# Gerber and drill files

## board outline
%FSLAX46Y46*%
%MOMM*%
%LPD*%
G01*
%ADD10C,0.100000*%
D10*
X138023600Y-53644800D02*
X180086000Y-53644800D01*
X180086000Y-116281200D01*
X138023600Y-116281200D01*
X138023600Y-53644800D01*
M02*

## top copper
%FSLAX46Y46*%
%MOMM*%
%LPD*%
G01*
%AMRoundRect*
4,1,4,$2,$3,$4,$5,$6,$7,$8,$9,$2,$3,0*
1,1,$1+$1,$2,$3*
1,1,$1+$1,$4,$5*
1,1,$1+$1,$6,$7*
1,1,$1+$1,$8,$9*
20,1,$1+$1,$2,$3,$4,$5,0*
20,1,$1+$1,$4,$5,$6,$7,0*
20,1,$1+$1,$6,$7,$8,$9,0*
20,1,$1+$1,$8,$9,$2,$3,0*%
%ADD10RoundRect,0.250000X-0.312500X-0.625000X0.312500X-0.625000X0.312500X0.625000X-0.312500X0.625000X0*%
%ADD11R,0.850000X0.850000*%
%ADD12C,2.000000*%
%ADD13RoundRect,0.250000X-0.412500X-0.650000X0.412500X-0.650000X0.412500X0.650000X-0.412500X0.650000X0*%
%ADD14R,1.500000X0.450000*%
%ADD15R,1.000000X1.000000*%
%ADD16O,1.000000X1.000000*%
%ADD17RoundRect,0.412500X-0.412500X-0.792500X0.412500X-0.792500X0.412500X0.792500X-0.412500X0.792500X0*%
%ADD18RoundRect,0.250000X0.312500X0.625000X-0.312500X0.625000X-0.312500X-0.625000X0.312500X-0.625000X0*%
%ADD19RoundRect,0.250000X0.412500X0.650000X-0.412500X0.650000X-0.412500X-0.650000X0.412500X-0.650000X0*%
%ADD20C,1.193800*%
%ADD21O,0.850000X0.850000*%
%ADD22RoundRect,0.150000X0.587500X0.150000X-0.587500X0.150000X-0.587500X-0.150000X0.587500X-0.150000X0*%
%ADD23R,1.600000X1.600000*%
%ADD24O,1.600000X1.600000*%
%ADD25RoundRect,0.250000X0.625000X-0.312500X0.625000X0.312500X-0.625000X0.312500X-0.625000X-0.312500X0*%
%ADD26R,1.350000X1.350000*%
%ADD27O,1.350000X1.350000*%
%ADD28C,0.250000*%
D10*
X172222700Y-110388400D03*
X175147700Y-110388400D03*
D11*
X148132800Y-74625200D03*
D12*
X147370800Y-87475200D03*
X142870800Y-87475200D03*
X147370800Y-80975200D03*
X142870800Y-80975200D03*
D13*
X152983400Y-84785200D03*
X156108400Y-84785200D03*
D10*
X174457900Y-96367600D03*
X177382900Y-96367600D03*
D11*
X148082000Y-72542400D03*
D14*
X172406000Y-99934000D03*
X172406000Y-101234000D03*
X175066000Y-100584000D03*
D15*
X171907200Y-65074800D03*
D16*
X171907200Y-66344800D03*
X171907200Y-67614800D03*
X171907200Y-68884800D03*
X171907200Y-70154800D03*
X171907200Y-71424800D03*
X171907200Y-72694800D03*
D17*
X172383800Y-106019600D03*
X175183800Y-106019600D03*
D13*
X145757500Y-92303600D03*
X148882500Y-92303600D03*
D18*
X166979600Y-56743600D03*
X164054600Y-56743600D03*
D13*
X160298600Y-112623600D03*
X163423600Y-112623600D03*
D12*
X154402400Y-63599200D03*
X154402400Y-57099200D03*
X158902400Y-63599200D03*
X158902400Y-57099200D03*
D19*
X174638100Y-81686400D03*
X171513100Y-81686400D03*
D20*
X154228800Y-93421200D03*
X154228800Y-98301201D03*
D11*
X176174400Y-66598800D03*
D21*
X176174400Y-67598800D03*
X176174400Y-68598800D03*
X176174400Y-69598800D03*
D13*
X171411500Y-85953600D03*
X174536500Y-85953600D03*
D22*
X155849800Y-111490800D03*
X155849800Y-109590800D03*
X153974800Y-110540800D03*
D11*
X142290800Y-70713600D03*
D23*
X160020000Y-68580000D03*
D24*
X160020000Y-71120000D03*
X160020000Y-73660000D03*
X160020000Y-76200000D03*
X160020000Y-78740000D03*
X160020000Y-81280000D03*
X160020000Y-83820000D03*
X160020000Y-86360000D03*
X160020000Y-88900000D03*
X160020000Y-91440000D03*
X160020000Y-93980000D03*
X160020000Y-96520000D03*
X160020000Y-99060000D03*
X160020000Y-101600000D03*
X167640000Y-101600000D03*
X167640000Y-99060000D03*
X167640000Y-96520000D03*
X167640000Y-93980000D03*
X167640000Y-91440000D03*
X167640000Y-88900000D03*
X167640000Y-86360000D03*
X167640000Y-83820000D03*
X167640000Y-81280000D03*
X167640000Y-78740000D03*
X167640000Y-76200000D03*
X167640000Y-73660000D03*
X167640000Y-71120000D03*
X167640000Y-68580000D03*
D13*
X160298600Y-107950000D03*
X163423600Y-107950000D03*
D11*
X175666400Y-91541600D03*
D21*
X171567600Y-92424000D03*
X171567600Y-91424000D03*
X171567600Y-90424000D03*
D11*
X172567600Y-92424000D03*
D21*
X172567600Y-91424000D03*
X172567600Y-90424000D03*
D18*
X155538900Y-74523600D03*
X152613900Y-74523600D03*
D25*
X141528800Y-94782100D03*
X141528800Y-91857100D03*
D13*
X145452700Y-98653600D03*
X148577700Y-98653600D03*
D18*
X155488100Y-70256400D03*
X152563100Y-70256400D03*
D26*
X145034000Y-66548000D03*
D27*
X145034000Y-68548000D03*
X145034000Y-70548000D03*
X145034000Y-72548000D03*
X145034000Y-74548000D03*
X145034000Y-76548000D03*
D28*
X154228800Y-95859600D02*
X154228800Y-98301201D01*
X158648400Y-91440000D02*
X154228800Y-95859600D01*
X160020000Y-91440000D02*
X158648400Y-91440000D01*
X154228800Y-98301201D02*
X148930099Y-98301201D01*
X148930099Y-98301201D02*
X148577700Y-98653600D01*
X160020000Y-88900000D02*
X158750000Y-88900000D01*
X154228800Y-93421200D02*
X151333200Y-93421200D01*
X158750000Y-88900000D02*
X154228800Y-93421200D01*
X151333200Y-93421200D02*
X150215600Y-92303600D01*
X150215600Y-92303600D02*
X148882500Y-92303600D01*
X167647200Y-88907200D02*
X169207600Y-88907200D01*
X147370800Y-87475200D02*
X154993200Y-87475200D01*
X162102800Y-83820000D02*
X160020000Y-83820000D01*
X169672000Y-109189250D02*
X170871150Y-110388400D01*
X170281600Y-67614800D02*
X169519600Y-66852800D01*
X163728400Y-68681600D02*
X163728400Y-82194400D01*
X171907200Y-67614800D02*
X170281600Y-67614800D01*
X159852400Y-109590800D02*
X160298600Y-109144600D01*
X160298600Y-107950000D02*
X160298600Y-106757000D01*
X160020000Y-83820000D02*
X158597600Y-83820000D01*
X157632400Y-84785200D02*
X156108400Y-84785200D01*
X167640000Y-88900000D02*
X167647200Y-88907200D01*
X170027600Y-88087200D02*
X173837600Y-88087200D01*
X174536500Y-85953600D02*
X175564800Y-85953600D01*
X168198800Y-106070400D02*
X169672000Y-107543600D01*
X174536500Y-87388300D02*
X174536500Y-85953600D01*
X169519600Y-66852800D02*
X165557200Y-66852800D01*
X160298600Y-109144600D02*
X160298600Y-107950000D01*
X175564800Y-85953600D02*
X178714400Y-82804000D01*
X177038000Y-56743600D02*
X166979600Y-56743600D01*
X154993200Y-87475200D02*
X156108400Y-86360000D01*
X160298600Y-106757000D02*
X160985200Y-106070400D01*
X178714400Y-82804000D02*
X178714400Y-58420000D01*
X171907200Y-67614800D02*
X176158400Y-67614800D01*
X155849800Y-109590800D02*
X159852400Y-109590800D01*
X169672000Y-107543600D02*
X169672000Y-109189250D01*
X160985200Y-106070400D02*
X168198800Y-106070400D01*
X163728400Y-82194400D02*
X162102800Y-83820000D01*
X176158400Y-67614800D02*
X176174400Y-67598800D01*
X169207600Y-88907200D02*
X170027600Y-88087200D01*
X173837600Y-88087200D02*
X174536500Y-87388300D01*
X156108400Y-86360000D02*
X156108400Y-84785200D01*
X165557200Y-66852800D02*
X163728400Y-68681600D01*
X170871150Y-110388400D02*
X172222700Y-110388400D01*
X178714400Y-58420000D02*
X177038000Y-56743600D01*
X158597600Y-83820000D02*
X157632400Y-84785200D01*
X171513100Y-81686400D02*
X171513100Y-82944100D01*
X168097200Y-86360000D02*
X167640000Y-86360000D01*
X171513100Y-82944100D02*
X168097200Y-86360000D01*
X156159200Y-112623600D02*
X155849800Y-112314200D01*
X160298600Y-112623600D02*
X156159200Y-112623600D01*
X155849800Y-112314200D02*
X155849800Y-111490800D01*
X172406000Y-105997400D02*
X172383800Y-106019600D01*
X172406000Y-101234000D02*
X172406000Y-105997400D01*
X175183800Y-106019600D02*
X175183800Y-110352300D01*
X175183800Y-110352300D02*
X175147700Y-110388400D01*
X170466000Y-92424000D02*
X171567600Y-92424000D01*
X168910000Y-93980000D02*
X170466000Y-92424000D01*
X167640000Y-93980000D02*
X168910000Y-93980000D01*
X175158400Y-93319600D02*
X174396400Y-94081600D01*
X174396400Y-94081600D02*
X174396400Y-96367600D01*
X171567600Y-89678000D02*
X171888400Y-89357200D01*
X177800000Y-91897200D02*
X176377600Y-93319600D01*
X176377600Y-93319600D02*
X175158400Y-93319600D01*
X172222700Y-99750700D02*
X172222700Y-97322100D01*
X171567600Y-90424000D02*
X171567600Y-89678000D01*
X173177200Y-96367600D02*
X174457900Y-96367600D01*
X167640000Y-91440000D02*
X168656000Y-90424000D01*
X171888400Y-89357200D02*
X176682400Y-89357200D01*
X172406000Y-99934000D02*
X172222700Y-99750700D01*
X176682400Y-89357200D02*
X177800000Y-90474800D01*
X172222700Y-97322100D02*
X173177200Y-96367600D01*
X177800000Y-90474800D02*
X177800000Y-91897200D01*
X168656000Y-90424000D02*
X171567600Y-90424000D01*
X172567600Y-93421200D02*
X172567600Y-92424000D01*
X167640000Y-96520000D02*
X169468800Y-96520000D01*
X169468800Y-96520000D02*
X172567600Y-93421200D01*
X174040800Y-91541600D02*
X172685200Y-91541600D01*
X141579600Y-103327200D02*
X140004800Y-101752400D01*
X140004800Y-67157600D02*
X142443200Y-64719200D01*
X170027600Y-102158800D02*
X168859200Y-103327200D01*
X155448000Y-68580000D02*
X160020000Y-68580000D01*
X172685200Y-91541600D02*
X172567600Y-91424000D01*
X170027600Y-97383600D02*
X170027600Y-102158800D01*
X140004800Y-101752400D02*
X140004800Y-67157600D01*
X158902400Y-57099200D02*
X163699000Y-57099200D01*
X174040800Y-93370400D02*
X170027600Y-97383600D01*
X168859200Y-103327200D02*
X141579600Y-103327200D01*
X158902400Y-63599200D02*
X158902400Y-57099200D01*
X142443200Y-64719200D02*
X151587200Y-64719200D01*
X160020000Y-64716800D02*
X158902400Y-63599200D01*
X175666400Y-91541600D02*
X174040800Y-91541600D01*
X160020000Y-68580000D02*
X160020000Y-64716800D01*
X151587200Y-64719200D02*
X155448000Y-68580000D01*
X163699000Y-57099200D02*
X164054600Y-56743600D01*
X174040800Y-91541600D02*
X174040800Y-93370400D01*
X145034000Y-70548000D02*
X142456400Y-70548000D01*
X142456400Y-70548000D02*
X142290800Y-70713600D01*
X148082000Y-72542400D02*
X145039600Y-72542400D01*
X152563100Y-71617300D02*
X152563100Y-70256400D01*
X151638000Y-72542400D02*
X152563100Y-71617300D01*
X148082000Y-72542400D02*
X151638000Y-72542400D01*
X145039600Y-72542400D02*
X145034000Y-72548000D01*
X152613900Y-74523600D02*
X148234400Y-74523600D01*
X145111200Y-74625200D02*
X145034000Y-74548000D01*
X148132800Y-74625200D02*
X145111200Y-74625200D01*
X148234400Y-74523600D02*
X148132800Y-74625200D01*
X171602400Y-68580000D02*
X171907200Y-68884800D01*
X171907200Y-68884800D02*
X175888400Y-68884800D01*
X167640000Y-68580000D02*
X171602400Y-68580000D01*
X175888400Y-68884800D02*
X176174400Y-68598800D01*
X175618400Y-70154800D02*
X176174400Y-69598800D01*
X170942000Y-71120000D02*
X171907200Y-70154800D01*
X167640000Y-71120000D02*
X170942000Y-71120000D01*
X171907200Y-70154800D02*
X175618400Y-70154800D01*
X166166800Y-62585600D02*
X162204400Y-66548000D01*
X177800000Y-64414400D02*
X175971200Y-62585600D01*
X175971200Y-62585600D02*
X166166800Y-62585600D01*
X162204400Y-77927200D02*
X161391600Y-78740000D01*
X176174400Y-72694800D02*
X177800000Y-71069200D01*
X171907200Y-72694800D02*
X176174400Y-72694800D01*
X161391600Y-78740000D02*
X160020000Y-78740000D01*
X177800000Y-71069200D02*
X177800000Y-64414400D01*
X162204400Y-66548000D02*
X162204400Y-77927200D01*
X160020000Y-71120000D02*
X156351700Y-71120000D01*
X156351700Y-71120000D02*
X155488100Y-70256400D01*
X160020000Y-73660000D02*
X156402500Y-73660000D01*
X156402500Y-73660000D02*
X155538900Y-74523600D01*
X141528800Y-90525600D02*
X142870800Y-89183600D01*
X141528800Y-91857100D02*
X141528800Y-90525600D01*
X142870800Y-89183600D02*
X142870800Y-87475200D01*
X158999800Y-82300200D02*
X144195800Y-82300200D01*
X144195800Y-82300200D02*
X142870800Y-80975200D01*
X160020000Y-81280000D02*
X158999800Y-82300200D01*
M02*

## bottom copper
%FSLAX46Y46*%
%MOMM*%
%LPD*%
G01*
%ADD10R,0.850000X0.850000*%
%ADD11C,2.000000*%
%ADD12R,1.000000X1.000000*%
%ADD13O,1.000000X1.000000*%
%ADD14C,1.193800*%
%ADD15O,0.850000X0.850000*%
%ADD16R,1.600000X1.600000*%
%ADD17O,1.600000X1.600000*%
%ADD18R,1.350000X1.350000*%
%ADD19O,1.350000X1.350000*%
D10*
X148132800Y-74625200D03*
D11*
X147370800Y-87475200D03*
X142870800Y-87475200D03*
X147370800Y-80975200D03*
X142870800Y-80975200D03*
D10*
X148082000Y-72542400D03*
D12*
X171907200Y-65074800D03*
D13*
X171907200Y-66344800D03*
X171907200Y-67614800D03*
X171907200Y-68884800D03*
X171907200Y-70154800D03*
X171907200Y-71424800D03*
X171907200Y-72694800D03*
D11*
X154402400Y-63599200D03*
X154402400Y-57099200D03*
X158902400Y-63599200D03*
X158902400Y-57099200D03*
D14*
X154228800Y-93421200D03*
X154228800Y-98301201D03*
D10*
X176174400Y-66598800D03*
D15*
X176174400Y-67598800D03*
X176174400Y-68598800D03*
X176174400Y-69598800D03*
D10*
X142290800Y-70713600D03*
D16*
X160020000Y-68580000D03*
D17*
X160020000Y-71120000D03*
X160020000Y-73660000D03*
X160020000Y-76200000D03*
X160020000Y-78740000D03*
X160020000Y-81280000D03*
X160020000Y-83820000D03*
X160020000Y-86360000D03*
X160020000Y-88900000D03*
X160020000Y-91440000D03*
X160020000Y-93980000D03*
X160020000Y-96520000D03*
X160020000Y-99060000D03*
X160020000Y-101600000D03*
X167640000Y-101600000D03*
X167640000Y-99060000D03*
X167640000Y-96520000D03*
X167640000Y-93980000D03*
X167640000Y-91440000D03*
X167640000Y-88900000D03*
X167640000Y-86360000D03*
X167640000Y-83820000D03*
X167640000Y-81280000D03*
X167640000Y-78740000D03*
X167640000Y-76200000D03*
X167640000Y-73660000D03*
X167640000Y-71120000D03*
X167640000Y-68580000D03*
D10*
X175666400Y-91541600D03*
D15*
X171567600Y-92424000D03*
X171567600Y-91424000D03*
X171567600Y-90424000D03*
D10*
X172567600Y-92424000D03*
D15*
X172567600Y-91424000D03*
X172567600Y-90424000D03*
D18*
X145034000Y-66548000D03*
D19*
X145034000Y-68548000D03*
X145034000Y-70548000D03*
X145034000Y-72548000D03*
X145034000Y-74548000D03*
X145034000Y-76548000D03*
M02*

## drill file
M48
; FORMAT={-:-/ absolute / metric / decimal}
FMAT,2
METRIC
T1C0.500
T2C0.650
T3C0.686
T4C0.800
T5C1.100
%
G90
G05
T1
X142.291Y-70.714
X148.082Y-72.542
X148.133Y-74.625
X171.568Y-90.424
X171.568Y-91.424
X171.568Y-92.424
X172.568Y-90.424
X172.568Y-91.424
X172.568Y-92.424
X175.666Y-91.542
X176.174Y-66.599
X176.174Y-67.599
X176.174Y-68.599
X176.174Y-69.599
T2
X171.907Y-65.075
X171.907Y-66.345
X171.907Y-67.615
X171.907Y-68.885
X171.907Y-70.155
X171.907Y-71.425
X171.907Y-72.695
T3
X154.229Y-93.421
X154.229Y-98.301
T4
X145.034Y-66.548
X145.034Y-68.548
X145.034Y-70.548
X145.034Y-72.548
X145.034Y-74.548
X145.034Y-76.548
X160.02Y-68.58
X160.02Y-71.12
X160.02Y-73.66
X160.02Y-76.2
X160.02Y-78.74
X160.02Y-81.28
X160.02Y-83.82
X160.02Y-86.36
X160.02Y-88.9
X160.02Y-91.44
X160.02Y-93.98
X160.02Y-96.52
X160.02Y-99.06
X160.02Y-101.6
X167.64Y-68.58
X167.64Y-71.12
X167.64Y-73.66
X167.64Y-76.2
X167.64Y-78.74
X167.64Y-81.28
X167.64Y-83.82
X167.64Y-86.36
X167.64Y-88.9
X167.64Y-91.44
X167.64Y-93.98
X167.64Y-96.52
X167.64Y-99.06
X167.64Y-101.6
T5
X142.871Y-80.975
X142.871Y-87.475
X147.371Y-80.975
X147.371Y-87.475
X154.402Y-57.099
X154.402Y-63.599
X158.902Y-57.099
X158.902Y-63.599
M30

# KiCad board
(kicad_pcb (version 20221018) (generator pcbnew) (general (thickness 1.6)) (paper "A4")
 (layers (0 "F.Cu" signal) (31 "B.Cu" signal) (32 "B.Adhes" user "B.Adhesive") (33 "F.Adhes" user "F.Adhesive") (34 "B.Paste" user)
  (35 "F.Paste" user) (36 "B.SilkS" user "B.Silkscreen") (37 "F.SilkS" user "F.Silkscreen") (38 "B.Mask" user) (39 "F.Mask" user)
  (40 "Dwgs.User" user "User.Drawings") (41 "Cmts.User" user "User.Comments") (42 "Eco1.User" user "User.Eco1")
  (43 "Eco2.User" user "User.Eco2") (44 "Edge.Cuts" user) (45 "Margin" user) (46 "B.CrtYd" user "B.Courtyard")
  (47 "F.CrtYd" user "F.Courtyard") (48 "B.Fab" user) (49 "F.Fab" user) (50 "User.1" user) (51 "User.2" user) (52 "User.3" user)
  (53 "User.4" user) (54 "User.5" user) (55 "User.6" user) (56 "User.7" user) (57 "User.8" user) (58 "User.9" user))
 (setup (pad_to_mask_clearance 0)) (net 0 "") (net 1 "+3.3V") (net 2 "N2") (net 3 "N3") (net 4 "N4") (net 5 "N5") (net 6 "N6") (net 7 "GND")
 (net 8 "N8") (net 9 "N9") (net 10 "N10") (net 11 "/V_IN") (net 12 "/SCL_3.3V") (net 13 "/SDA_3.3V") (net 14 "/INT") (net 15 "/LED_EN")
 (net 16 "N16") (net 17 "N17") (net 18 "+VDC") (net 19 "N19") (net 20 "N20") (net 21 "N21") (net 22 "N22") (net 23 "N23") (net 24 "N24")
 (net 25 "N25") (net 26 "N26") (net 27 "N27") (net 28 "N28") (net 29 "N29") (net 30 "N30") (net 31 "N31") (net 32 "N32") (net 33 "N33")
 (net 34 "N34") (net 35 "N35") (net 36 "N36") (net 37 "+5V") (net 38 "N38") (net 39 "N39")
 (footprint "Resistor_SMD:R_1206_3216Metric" (layer "F.Cu") (at 173.6852 110.3884)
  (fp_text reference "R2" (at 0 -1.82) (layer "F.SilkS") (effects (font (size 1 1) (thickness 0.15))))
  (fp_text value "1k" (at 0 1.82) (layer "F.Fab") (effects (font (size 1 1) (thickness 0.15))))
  (pad "1" smd roundrect (at -1.4625 0) (size 1.125 1.75) (layers "F.Cu" "F.Paste" "F.Mask") (roundrect_rratio 0.222222) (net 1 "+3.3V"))
  (pad "2" smd roundrect (at 1.4625 0) (size 1.125 1.75) (layers "F.Cu" "F.Paste" "F.Mask") (roundrect_rratio 0.222222) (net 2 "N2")))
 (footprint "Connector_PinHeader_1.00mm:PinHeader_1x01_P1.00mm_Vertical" (layer "F.Cu") (at 148.1328 74.6252)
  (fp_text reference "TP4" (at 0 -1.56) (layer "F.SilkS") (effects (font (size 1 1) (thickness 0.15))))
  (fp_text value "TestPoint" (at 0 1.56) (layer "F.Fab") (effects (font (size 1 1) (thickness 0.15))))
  (pad "1" thru_hole rect (at 0 0) (size 0.85 0.85) (drill 0.5) (layers "*.Cu" "*.Mask") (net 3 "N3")))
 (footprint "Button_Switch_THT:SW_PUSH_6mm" (layer "F.Cu") (at 147.3708 80.9752 -90)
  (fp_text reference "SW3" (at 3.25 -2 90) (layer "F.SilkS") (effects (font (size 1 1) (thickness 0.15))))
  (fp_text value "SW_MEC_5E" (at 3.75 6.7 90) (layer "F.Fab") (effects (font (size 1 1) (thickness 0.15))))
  (pad "1" thru_hole circle (at 6.5 0) (size 2 2) (drill 1.1) (layers "*.Cu" "*.Mask") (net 1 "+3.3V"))
  (pad "2" thru_hole circle (at 6.5 4.5) (size 2 2) (drill 1.1) (layers "*.Cu" "*.Mask") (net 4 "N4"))
  (pad "3" thru_hole circle (at 0 0) (size 2 2) (drill 1.1) (layers "*.Cu" "*.Mask") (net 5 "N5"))
  (pad "4" thru_hole circle (at 0 4.5) (size 2 2) (drill 1.1) (layers "*.Cu" "*.Mask") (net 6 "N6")))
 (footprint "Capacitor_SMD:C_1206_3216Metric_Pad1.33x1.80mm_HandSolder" (layer "F.Cu") (at 154.5459 84.7852)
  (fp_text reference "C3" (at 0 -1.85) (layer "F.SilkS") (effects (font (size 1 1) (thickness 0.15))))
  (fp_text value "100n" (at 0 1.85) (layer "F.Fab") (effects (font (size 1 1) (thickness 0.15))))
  (pad "1" smd roundrect (at -1.5625 0) (size 1.325 1.8) (layers "F.Cu" "F.Paste" "F.Mask") (roundrect_rratio 0.188679) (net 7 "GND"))
  (pad "2" smd roundrect (at 1.5625 0) (size 1.325 1.8) (layers "F.Cu" "F.Paste" "F.Mask") (roundrect_rratio 0.188679) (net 1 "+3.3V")))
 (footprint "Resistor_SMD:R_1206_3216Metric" (layer "F.Cu") (at 175.9204 96.3676)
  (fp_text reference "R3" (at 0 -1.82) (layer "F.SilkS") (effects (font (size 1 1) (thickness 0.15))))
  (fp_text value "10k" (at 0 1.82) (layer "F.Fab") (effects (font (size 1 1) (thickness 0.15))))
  (pad "1" smd roundrect (at -1.4625 0) (size 1.125 1.75) (layers "F.Cu" "F.Paste" "F.Mask") (roundrect_rratio 0.222222) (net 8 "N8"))
  (pad "2" smd roundrect (at 1.4625 0) (size 1.125 1.75) (layers "F.Cu" "F.Paste" "F.Mask") (roundrect_rratio 0.222222) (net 7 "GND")))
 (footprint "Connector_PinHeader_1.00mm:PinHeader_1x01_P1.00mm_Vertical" (layer "F.Cu") (at 148.082 72.5424)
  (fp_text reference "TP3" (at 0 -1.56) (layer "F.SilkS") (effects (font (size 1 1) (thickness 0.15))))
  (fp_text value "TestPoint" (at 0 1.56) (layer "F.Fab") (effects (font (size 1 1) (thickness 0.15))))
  (pad "1" thru_hole rect (at 0 0) (size 0.85 0.85) (drill 0.5) (layers "*.Cu" "*.Mask") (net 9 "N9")))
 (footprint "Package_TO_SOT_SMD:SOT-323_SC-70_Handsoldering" (layer "F.Cu") (at 173.736 100.584)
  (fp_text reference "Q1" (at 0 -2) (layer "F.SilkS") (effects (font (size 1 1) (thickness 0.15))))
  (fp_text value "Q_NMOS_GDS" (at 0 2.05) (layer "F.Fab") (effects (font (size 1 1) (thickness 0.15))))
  (pad "1" smd rect (at -1.33 -0.65 270) (size 0.45 1.5) (layers "F.Cu" "F.Paste" "F.Mask") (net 8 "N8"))
  (pad "2" smd rect (at -1.33 0.65 270) (size 0.45 1.5) (layers "F.Cu" "F.Paste" "F.Mask") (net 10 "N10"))
  (pad "3" smd rect (at 1.33 0 270) (size 0.45 1.5) (layers "F.Cu" "F.Paste" "F.Mask") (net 7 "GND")))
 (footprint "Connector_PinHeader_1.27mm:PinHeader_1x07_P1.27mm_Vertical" (layer "F.Cu") (at 171.9072 65.0748)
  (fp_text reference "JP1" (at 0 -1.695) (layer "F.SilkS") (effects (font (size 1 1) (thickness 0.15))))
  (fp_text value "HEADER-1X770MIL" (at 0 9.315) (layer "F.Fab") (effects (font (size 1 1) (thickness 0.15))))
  (pad "1" thru_hole rect (at 0 0) (size 1 1) (drill 0.65) (layers "*.Cu" "*.Mask") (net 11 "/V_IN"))
  (pad "2" thru_hole oval (at 0 1.27) (size 1 1) (drill 0.65) (layers "*.Cu" "*.Mask") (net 7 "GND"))
  (pad "3" thru_hole oval (at 0 2.54) (size 1 1) (drill 0.65) (layers "*.Cu" "*.Mask") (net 1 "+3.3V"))
  (pad "4" thru_hole oval (at 0 3.81) (size 1 1) (drill 0.65) (layers "*.Cu" "*.Mask") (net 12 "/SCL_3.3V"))
  (pad "5" thru_hole oval (at 0 5.08) (size 1 1) (drill 0.65) (layers "*.Cu" "*.Mask") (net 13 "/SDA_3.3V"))
  (pad "6" thru_hole oval (at 0 6.35) (size 1 1) (drill 0.65) (layers "*.Cu" "*.Mask") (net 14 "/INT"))
  (pad "7" thru_hole oval (at 0 7.62) (size 1 1) (drill 0.65) (layers "*.Cu" "*.Mask") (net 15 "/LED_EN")))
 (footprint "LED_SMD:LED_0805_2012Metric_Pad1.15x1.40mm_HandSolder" (layer "F.Cu") (at 173.7868 106.0196)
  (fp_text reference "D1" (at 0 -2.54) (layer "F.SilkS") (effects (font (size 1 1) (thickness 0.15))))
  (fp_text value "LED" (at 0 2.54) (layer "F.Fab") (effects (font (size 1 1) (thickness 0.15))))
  (pad "1" smd roundrect (at -1.403 0) (size 1.65 2.41) (layers "F.Cu" "F.Paste" "F.Mask") (roundrect_rratio 0.25) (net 10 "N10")
   (thermal_bridge_angle 45))
  (pad "2" smd roundrect (at 1.397 0) (size 1.65 2.41) (layers "F.Cu" "F.Paste" "F.Mask") (roundrect_rratio 0.25) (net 2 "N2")
   (thermal_bridge_angle 45)))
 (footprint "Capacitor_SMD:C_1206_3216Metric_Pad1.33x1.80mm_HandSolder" (layer "F.Cu") (at 147.32 92.3036)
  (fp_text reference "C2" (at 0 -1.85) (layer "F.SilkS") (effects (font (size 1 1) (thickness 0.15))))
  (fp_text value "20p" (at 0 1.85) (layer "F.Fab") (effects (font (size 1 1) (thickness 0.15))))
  (pad "1" smd roundrect (at -1.5625 0) (size 1.325 1.8) (layers "F.Cu" "F.Paste" "F.Mask") (roundrect_rratio 0.188679) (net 7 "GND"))
  (pad "2" smd roundrect (at 1.5625 0) (size 1.325 1.8) (layers "F.Cu" "F.Paste" "F.Mask") (roundrect_rratio 0.188679) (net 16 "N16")))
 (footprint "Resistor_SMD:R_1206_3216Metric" (layer "F.Cu") (at 165.5171 56.7436 180)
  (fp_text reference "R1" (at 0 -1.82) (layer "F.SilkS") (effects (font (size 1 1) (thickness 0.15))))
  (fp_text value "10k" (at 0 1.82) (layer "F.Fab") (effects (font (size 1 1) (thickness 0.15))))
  (pad "1" smd roundrect (at -1.4625 0 180) (size 1.125 1.75) (layers "F.Cu" "F.Paste" "F.Mask") (roundrect_rratio 0.222222) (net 1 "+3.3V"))
  (pad "2" smd roundrect (at 1.4625 0 180) (size 1.125 1.75) (layers "F.Cu" "F.Paste" "F.Mask") (roundrect_rratio 0.222222) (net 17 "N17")))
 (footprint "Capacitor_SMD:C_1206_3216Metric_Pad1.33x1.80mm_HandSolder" (layer "F.Cu") (at 161.8611 112.6236)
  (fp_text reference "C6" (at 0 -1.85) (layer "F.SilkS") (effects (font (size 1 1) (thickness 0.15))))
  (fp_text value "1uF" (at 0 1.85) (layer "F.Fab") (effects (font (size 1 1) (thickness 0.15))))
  (pad "1" smd roundrect (at -1.5625 0) (size 1.325 1.8) (layers "F.Cu" "F.Paste" "F.Mask") (roundrect_rratio 0.188679) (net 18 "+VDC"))
  (pad "2" smd roundrect (at 1.5625 0) (size 1.325 1.8) (layers "F.Cu" "F.Paste" "F.Mask") (roundrect_rratio 0.188679) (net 7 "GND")))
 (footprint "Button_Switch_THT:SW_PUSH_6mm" (layer "F.Cu") (at 154.4024 63.5992 90)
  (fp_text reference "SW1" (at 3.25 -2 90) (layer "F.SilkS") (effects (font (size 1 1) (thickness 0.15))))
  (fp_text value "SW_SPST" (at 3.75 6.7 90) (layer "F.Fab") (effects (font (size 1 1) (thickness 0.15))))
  (pad "1" thru_hole circle (at 0 0 180) (size 2 2) (drill 1.1) (layers "*.Cu" "*.Mask") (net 7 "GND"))
  (pad "1" thru_hole circle (at 6.5 0 180) (size 2 2) (drill 1.1) (layers "*.Cu" "*.Mask") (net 7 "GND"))
  (pad "2" thru_hole circle (at 0 4.5 180) (size 2 2) (drill 1.1) (layers "*.Cu" "*.Mask") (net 17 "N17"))
  (pad "2" thru_hole circle (at 6.5 4.5 180) (size 2 2) (drill 1.1) (layers "*.Cu" "*.Mask") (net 17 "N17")))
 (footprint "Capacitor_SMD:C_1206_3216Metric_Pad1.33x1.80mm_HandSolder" (layer "F.Cu") (at 173.0756 81.6864 180)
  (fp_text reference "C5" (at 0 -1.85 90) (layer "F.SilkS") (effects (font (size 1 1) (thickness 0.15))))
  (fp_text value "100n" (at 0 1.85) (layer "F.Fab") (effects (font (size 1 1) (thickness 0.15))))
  (pad "1" smd roundrect (at -1.5625 0 180) (size 1.325 1.8) (layers "F.Cu" "F.Paste" "F.Mask") (roundrect_rratio 0.188679) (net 7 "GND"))
  (pad "2" smd roundrect (at 1.5625 0 180) (size 1.325 1.8) (layers "F.Cu" "F.Paste" "F.Mask") (roundrect_rratio 0.188679) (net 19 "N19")))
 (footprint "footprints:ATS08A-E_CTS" (layer "F.Cu") (at 154.2288 93.4212 -90)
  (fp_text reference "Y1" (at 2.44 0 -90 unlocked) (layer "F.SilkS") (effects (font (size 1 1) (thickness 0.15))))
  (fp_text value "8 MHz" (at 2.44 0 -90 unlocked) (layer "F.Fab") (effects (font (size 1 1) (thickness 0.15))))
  (pad "1" thru_hole circle (at 0 0 270) (size 1.1938 1.1938) (drill 0.6858) (layers "*.Cu" "*.Mask") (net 16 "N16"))
  (pad "2" thru_hole circle (at 4.880001 0 270) (size 1.1938 1.1938) (drill 0.6858) (layers "*.Cu" "*.Mask") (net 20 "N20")))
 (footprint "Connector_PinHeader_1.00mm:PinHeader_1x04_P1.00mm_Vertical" (layer "F.Cu") (at 176.1744 66.5988)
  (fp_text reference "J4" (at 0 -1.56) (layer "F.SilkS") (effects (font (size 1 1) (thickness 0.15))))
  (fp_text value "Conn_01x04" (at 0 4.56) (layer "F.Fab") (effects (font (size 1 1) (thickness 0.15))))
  (pad "1" thru_hole rect (at 0 0) (size 0.85 0.85) (drill 0.5) (layers "*.Cu" "*.Mask") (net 7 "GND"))
  (pad "2" thru_hole oval (at 0 1) (size 0.85 0.85) (drill 0.5) (layers "*.Cu" "*.Mask") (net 1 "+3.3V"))
  (pad "3" thru_hole oval (at 0 2) (size 0.85 0.85) (drill 0.5) (layers "*.Cu" "*.Mask") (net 12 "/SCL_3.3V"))
  (pad "4" thru_hole oval (at 0 3) (size 0.85 0.85) (drill 0.5) (layers "*.Cu" "*.Mask") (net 13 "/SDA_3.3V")))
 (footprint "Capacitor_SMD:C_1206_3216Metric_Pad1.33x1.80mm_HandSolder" (layer "F.Cu") (at 172.974 85.9536)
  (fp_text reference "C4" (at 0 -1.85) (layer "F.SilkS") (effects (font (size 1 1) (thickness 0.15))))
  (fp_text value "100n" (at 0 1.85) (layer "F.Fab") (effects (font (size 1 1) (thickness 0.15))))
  (pad "1" smd roundrect (at -1.5625 0) (size 1.325 1.8) (layers "F.Cu" "F.Paste" "F.Mask") (roundrect_rratio 0.188679) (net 7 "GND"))
  (pad "2" smd roundrect (at 1.5625 0) (size 1.325 1.8) (layers "F.Cu" "F.Paste" "F.Mask") (roundrect_rratio 0.188679) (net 1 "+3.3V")))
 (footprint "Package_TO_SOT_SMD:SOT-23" (layer "F.Cu") (at 154.9123 110.5408 180)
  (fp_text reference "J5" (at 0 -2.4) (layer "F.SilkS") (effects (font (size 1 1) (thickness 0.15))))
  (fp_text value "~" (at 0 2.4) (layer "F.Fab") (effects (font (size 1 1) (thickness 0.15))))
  (pad "1" smd roundrect (at -0.9375 -0.95 180) (size 1.475 0.6) (layers "F.Cu" "F.Paste" "F.Mask") (roundrect_rratio 0.25) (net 18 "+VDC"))
  (pad "2" smd roundrect (at -0.9375 0.95 180) (size 1.475 0.6) (layers "F.Cu" "F.Paste" "F.Mask") (roundrect_rratio 0.25) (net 1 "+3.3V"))
  (pad "3" smd roundrect (at 0.9375 0 180) (size 1.475 0.6) (layers "F.Cu" "F.Paste" "F.Mask") (roundrect_rratio 0.25) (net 7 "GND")))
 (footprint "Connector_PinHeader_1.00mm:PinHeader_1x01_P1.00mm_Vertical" (layer "F.Cu") (at 142.2908 70.7136)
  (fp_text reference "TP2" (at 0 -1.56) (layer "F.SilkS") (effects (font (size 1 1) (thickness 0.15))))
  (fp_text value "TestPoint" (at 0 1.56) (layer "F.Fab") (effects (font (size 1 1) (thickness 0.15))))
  (pad "1" thru_hole rect (at 0 0) (size 0.85 0.85) (drill 0.5) (layers "*.Cu" "*.Mask") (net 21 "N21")))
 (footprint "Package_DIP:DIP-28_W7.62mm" (layer "F.Cu") (at 160.02 68.58)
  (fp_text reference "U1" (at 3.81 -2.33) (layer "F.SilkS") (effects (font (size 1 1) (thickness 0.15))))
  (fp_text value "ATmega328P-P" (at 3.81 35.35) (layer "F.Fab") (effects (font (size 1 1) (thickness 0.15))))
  (pad "1" thru_hole rect (at 0 0) (size 1.6 1.6) (drill 0.8) (layers "*.Cu" "*.Mask") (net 17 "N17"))
  (pad "2" thru_hole oval (at 0 2.54) (size 1.6 1.6) (drill 0.8) (layers "*.Cu" "*.Mask") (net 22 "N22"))
  (pad "3" thru_hole oval (at 0 5.08) (size 1.6 1.6) (drill 0.8) (layers "*.Cu" "*.Mask") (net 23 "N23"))
  (pad "4" thru_hole oval (at 0 7.62) (size 1.6 1.6) (drill 0.8) (layers "*.Cu" "*.Mask") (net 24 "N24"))
  (pad "5" thru_hole oval (at 0 10.16) (size 1.6 1.6) (drill 0.8) (layers "*.Cu" "*.Mask") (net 15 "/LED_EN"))
  (pad "6" thru_hole oval (at 0 12.7) (size 1.6 1.6) (drill 0.8) (layers "*.Cu" "*.Mask") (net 6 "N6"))
  (pad "7" thru_hole oval (at 0 15.24) (size 1.6 1.6) (drill 0.8) (layers "*.Cu" "*.Mask") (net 1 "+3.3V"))
  (pad "8" thru_hole oval (at 0 17.78) (size 1.6 1.6) (drill 0.8) (layers "*.Cu" "*.Mask") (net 7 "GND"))
  (pad "9" thru_hole oval (at 0 20.32) (size 1.6 1.6) (drill 0.8) (layers "*.Cu" "*.Mask") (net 16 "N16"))
  (pad "10" thru_hole oval (at 0 22.86) (size 1.6 1.6) (drill 0.8) (layers "*.Cu" "*.Mask") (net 20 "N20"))
  (pad "11" thru_hole oval (at 0 25.4) (size 1.6 1.6) (drill 0.8) (layers "*.Cu" "*.Mask") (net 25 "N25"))
  (pad "12" thru_hole oval (at 0 27.94) (size 1.6 1.6) (drill 0.8) (layers "*.Cu" "*.Mask") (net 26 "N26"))
  (pad "13" thru_hole oval (at 0 30.48) (size 1.6 1.6) (drill 0.8) (layers "*.Cu" "*.Mask") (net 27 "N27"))
  (pad "14" thru_hole oval (at 0 33.02) (size 1.6 1.6) (drill 0.8) (layers "*.Cu" "*.Mask") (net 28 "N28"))
  (pad "15" thru_hole oval (at 7.62 33.02) (size 1.6 1.6) (drill 0.8) (layers "*.Cu" "*.Mask") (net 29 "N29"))
  (pad "16" thru_hole oval (at 7.62 30.48) (size 1.6 1.6) (drill 0.8) (layers "*.Cu" "*.Mask") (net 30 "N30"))
  (pad "17" thru_hole oval (at 7.62 27.94) (size 1.6 1.6) (drill 0.8) (layers "*.Cu" "*.Mask") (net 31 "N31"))
  (pad "18" thru_hole oval (at 7.62 25.4) (size 1.6 1.6) (drill 0.8) (layers "*.Cu" "*.Mask") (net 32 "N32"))
  (pad "19" thru_hole oval (at 7.62 22.86) (size 1.6 1.6) (drill 0.8) (layers "*.Cu" "*.Mask") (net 8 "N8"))
  (pad "20" thru_hole oval (at 7.62 20.32) (size 1.6 1.6) (drill 0.8) (layers "*.Cu" "*.Mask") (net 1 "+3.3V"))
  (pad "21" thru_hole oval (at 7.62 17.78) (size 1.6 1.6) (drill 0.8) (layers "*.Cu" "*.Mask") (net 19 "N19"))
  (pad "22" thru_hole oval (at 7.62 15.24) (size 1.6 1.6) (drill 0.8) (layers "*.Cu" "*.Mask") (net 7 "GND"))
  (pad "23" thru_hole oval (at 7.62 12.7) (size 1.6 1.6) (drill 0.8) (layers "*.Cu" "*.Mask") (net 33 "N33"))
  (pad "24" thru_hole oval (at 7.62 10.16) (size 1.6 1.6) (drill 0.8) (layers "*.Cu" "*.Mask") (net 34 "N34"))
  (pad "25" thru_hole oval (at 7.62 7.62) (size 1.6 1.6) (drill 0.8) (layers "*.Cu" "*.Mask") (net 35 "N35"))
  (pad "26" thru_hole oval (at 7.62 5.08) (size 1.6 1.6) (drill 0.8) (layers "*.Cu" "*.Mask") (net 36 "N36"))
  (pad "27" thru_hole oval (at 7.62 2.54) (size 1.6 1.6) (drill 0.8) (layers "*.Cu" "*.Mask") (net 13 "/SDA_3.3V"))
  (pad "28" thru_hole oval (at 7.62 0) (size 1.6 1.6) (drill 0.8) (layers "*.Cu" "*.Mask") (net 12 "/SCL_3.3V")))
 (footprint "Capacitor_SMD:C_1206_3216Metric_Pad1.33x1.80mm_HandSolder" (layer "F.Cu") (at 161.8611 107.95)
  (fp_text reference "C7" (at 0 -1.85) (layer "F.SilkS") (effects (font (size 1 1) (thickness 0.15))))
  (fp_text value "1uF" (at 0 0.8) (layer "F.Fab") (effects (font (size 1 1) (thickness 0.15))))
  (pad "1" smd roundrect (at -1.5625 0) (size 1.325 1.8) (layers "F.Cu" "F.Paste" "F.Mask") (roundrect_rratio 0.188679) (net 1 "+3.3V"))
  (pad "2" smd roundrect (at 1.5625 0) (size 1.325 1.8) (layers "F.Cu" "F.Paste" "F.Mask") (roundrect_rratio 0.188679) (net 7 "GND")))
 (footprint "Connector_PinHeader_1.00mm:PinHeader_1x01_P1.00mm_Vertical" (layer "F.Cu") (at 175.6664 91.5416)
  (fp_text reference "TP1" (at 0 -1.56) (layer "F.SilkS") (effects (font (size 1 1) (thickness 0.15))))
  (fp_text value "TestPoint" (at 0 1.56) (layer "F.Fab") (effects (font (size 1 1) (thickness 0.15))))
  (pad "1" thru_hole rect (at 0 0) (size 0.85 0.85) (drill 0.5) (layers "*.Cu" "*.Mask") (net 17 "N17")))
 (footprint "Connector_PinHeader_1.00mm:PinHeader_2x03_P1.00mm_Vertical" (layer "F.Cu") (at 172.5676 92.424 180)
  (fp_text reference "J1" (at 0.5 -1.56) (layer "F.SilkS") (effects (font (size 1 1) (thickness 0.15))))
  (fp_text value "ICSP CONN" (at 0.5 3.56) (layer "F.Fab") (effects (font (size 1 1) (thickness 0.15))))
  (pad "1" thru_hole oval (at 1 0 180) (size 0.85 0.85) (drill 0.5) (layers "*.Cu" "*.Mask") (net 32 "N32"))
  (pad "2" thru_hole oval (at 1 1 180) (size 0.85 0.85) (drill 0.5) (layers "*.Cu" "*.Mask") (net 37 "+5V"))
  (pad "3" thru_hole oval (at 1 2 180) (size 0.85 0.85) (drill 0.5) (layers "*.Cu" "*.Mask") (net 8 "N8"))
  (pad "4" thru_hole rect (at 0 0 180) (size 0.85 0.85) (drill 0.5) (layers "*.Cu" "*.Mask") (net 31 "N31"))
  (pad "5" thru_hole oval (at 0 1 180) (size 0.85 0.85) (drill 0.5) (layers "*.Cu" "*.Mask") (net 17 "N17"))
  (pad "6" thru_hole oval (at 0 2 180) (size 0.85 0.85) (drill 0.5) (layers "*.Cu" "*.Mask") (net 7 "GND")))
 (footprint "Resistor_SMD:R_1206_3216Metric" (layer "F.Cu") (at 154.0764 74.5236 180)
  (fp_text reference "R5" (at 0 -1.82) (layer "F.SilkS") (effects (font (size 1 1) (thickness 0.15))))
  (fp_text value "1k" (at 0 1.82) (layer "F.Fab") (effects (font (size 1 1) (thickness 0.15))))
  (pad "1" smd roundrect (at -1.4625 0 180) (size 1.125 1.75) (layers "F.Cu" "F.Paste" "F.Mask") (roundrect_rratio 0.222222) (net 23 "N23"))
  (pad "2" smd roundrect (at 1.4625 0 180) (size 1.125 1.75) (layers "F.Cu" "F.Paste" "F.Mask") (roundrect_rratio 0.222222) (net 3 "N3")))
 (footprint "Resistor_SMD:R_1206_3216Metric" (layer "F.Cu") (at 141.5288 93.3196 90)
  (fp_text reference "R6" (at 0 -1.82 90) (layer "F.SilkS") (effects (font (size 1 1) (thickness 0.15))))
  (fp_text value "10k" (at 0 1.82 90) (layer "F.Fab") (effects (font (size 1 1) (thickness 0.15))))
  (pad "1" smd roundrect (at -1.4625 0 90) (size 1.125 1.75) (layers "F.Cu" "F.Paste" "F.Mask") (roundrect_rratio 0.222222) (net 7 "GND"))
  (pad "2" smd roundrect (at 1.4625 0 90) (size 1.125 1.75) (layers "F.Cu" "F.Paste" "F.Mask") (roundrect_rratio 0.222222) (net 4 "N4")))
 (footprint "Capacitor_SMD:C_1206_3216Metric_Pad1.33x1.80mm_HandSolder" (layer "F.Cu") (at 147.0152 98.6536)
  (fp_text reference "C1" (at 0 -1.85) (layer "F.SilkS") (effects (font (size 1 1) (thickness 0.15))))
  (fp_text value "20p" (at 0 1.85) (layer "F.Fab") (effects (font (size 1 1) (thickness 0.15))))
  (pad "1" smd roundrect (at -1.5625 0) (size 1.325 1.8) (layers "F.Cu" "F.Paste" "F.Mask") (roundrect_rratio 0.188679) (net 7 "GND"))
  (pad "2" smd roundrect (at 1.5625 0) (size 1.325 1.8) (layers "F.Cu" "F.Paste" "F.Mask") (roundrect_rratio 0.188679) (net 20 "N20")))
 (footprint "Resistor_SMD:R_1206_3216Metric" (layer "F.Cu") (at 154.0256 70.2564 180)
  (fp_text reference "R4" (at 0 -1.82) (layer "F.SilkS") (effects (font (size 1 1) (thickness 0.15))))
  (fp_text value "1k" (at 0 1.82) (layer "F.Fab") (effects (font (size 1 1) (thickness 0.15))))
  (pad "1" smd roundrect (at -1.4625 0 180) (size 1.125 1.75) (layers "F.Cu" "F.Paste" "F.Mask") (roundrect_rratio 0.222222) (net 22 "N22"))
  (pad "2" smd roundrect (at 1.4625 0 180) (size 1.125 1.75) (layers "F.Cu" "F.Paste" "F.Mask") (roundrect_rratio 0.222222) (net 9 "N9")))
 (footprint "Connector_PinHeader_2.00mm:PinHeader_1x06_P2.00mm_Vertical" (layer "F.Cu") (at 145.034 66.548)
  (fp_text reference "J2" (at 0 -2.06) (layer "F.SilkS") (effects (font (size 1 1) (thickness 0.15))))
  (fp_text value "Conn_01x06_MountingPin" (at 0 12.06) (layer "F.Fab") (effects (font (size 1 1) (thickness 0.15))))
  (pad "1" thru_hole rect (at 0 0) (size 1.35 1.35) (drill 0.8) (layers "*.Cu" "*.Mask") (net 7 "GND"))
  (pad "2" thru_hole oval (at 0 2) (size 1.35 1.35) (drill 0.8) (layers "*.Cu" "*.Mask") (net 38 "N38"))
  (pad "3" thru_hole oval (at 0 4) (size 1.35 1.35) (drill 0.8) (layers "*.Cu" "*.Mask") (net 21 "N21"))
  (pad "4" thru_hole oval (at 0 6) (size 1.35 1.35) (drill 0.8) (layers "*.Cu" "*.Mask") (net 9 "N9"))
  (pad "5" thru_hole oval (at 0 8) (size 1.35 1.35) (drill 0.8) (layers "*.Cu" "*.Mask") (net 3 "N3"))
  (pad "6" thru_hole oval (at 0 10) (size 1.35 1.35) (drill 0.8) (layers "*.Cu" "*.Mask") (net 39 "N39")))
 (gr_rect (start 138.0236 53.6448) (end 180.086 116.2812) (stroke (width 0.1) (type default)) (fill none) (layer "Edge.Cuts"))
 (segment (start 154.2288 95.8596) (end 154.2288 98.301201) (width 0.25) (layer "F.Cu") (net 20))
 (segment (start 158.6484 91.44) (end 154.2288 95.8596) (width 0.25) (layer "F.Cu") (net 20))
 (segment (start 160.02 91.44) (end 158.6484 91.44) (width 0.25) (layer "F.Cu") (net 20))
 (segment (start 154.2288 98.301201) (end 148.930099 98.301201) (width 0.25) (layer "F.Cu") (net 20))
 (segment (start 148.930099 98.301201) (end 148.5777 98.6536) (width 0.25) (layer "F.Cu") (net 20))
 (segment (start 160.02 88.9) (end 158.75 88.9) (width 0.25) (layer "F.Cu") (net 16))
 (segment (start 154.2288 93.4212) (end 151.3332 93.4212) (width 0.25) (layer "F.Cu") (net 16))
 (segment (start 158.75 88.9) (end 154.2288 93.4212) (width 0.25) (layer "F.Cu") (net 16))
 (segment (start 151.3332 93.4212) (end 150.2156 92.3036) (width 0.25) (layer "F.Cu") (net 16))
 (segment (start 150.2156 92.3036) (end 148.8825 92.3036) (width 0.25) (layer "F.Cu") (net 16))
 (segment (start 167.6472 88.9072) (end 169.2076 88.9072) (width 0.25) (layer "F.Cu") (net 1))
 (segment (start 147.3708 87.4752) (end 154.9932 87.4752) (width 0.25) (layer "F.Cu") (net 1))
 (segment (start 162.1028 83.82) (end 160.02 83.82) (width 0.25) (layer "F.Cu") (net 1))
 (segment (start 169.672 109.18925) (end 170.87115 110.3884) (width 0.25) (layer "F.Cu") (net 1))
 (segment (start 170.2816 67.6148) (end 169.5196 66.8528) (width 0.25) (layer "F.Cu") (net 1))
 (segment (start 163.7284 68.6816) (end 163.7284 82.1944) (width 0.25) (layer "F.Cu") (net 1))
 (segment (start 171.9072 67.6148) (end 170.2816 67.6148) (width 0.25) (layer "F.Cu") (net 1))
 (segment (start 159.8524 109.5908) (end 160.2986 109.1446) (width 0.25) (layer "F.Cu") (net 1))
 (segment (start 160.2986 107.95) (end 160.2986 106.757) (width 0.25) (layer "F.Cu") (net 1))
 (segment (start 160.02 83.82) (end 158.5976 83.82) (width 0.25) (layer "F.Cu") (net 1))
 (segment (start 157.6324 84.7852) (end 156.1084 84.7852) (width 0.25) (layer "F.Cu") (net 1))
 (segment (start 167.64 88.9) (end 167.6472 88.9072) (width 0.25) (layer "F.Cu") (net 1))
 (segment (start 170.0276 88.0872) (end 173.8376 88.0872) (width 0.25) (layer "F.Cu") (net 1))
 (segment (start 174.5365 85.9536) (end 175.5648 85.9536) (width 0.25) (layer "F.Cu") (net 1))
 (segment (start 168.1988 106.0704) (end 169.672 107.5436) (width 0.25) (layer "F.Cu") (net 1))
 (segment (start 174.5365 87.3883) (end 174.5365 85.9536) (width 0.25) (layer "F.Cu") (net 1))
 (segment (start 169.5196 66.8528) (end 165.5572 66.8528) (width 0.25) (layer "F.Cu") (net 1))
 (segment (start 160.2986 109.1446) (end 160.2986 107.95) (width 0.25) (layer "F.Cu") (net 1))
 (segment (start 175.5648 85.9536) (end 178.7144 82.804) (width 0.25) (layer "F.Cu") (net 1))
 (segment (start 177.038 56.7436) (end 166.9796 56.7436) (width 0.25) (layer "F.Cu") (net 1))
 (segment (start 154.9932 87.4752) (end 156.1084 86.36) (width 0.25) (layer "F.Cu") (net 1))
 (segment (start 160.2986 106.757) (end 160.9852 106.0704) (width 0.25) (layer "F.Cu") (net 1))
 (segment (start 178.7144 82.804) (end 178.7144 58.42) (width 0.25) (layer "F.Cu") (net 1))
 (segment (start 171.9072 67.6148) (end 176.1584 67.6148) (width 0.25) (layer "F.Cu") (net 1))
 (segment (start 155.8498 109.5908) (end 159.8524 109.5908) (width 0.25) (layer "F.Cu") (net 1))
 (segment (start 169.672 107.5436) (end 169.672 109.18925) (width 0.25) (layer "F.Cu") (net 1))
 (segment (start 160.9852 106.0704) (end 168.1988 106.0704) (width 0.25) (layer "F.Cu") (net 1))
 (segment (start 163.7284 82.1944) (end 162.1028 83.82) (width 0.25) (layer "F.Cu") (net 1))
 (segment (start 176.1584 67.6148) (end 176.1744 67.5988) (width 0.25) (layer "F.Cu") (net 1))
 (segment (start 169.2076 88.9072) (end 170.0276 88.0872) (width 0.25) (layer "F.Cu") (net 1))
 (segment (start 173.8376 88.0872) (end 174.5365 87.3883) (width 0.25) (layer "F.Cu") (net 1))
 (segment (start 156.1084 86.36) (end 156.1084 84.7852) (width 0.25) (layer "F.Cu") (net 1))
 (segment (start 165.5572 66.8528) (end 163.7284 68.6816) (width 0.25) (layer "F.Cu") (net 1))
 (segment (start 170.87115 110.3884) (end 172.2227 110.3884) (width 0.25) (layer "F.Cu") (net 1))
 (segment (start 178.7144 58.42) (end 177.038 56.7436) (width 0.25) (layer "F.Cu") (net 1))
 (segment (start 158.5976 83.82) (end 157.6324 84.7852) (width 0.25) (layer "F.Cu") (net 1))
 (segment (start 171.5131 81.6864) (end 171.5131 82.9441) (width 0.25) (layer "F.Cu") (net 19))
 (segment (start 168.0972 86.36) (end 167.64 86.36) (width 0.25) (layer "F.Cu") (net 19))
 (segment (start 171.5131 82.9441) (end 168.0972 86.36) (width 0.25) (layer "F.Cu") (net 19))
 (segment (start 156.1592 112.6236) (end 155.8498 112.3142) (width 0.25) (layer "F.Cu") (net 18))
 (segment (start 160.2986 112.6236) (end 156.1592 112.6236) (width 0.25) (layer "F.Cu") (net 18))
 (segment (start 155.8498 112.3142) (end 155.8498 111.4908) (width 0.25) (layer "F.Cu") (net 18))
 (segment (start 172.406 105.9974) (end 172.3838 106.0196) (width 0.25) (layer "F.Cu") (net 10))
 (segment (start 172.406 101.234) (end 172.406 105.9974) (width 0.25) (layer "F.Cu") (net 10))
 (segment (start 175.1838 106.0196) (end 175.1838 110.3523) (width 0.25) (layer "F.Cu") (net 2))
 (segment (start 175.1838 110.3523) (end 175.1477 110.3884) (width 0.25) (layer "F.Cu") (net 2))
 (segment (start 170.466 92.424) (end 171.5676 92.424) (width 0.25) (layer "F.Cu") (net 32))
 (segment (start 168.91 93.98) (end 170.466 92.424) (width 0.25) (layer "F.Cu") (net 32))
 (segment (start 167.64 93.98) (end 168.91 93.98) (width 0.25) (layer "F.Cu") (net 32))
 (segment (start 175.1584 93.3196) (end 174.3964 94.0816) (width 0.25) (layer "F.Cu") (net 8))
 (segment (start 174.3964 94.0816) (end 174.3964 96.3676) (width 0.25) (layer "F.Cu") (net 8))
 (segment (start 171.5676 89.678) (end 171.8884 89.3572) (width 0.25) (layer "F.Cu") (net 8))
 (segment (start 177.8 91.8972) (end 176.3776 93.3196) (width 0.25) (layer "F.Cu") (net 8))
 (segment (start 176.3776 93.3196) (end 175.1584 93.3196) (width 0.25) (layer "F.Cu") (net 8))
 (segment (start 172.2227 99.7507) (end 172.2227 97.3221) (width 0.25) (layer "F.Cu") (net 8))
 (segment (start 171.5676 90.424) (end 171.5676 89.678) (width 0.25) (layer "F.Cu") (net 8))
 (segment (start 173.1772 96.3676) (end 174.4579 96.3676) (width 0.25) (layer "F.Cu") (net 8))
 (segment (start 167.64 91.44) (end 168.656 90.424) (width 0.25) (layer "F.Cu") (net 8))
 (segment (start 171.8884 89.3572) (end 176.6824 89.3572) (width 0.25) (layer "F.Cu") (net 8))
 (segment (start 172.406 99.934) (end 172.2227 99.7507) (width 0.25) (layer "F.Cu") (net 8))
 (segment (start 176.6824 89.3572) (end 177.8 90.4748) (width 0.25) (layer "F.Cu") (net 8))
 (segment (start 172.2227 97.3221) (end 173.1772 96.3676) (width 0.25) (layer "F.Cu") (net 8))
 (segment (start 177.8 90.4748) (end 177.8 91.8972) (width 0.25) (layer "F.Cu") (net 8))
 (segment (start 168.656 90.424) (end 171.5676 90.424) (width 0.25) (layer "F.Cu") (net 8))
 (segment (start 172.5676 93.4212) (end 172.5676 92.424) (width 0.25) (layer "F.Cu") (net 31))
 (segment (start 167.64 96.52) (end 169.4688 96.52) (width 0.25) (layer "F.Cu") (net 31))
 (segment (start 169.4688 96.52) (end 172.5676 93.4212) (width 0.25) (layer "F.Cu") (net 31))
 (segment (start 174.0408 91.5416) (end 172.6852 91.5416) (width 0.25) (layer "F.Cu") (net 17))
 (segment (start 141.5796 103.3272) (end 140.0048 101.7524) (width 0.25) (layer "F.Cu") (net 17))
 (segment (start 140.0048 67.1576) (end 142.4432 64.7192) (width 0.25) (layer "F.Cu") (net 17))
 (segment (start 170.0276 102.1588) (end 168.8592 103.3272) (width 0.25) (layer "F.Cu") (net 17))
 (segment (start 155.448 68.58) (end 160.02 68.58) (width 0.25) (layer "F.Cu") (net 17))
 (segment (start 172.6852 91.5416) (end 172.5676 91.424) (width 0.25) (layer "F.Cu") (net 17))
 (segment (start 170.0276 97.3836) (end 170.0276 102.1588) (width 0.25) (layer "F.Cu") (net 17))
 (segment (start 140.0048 101.7524) (end 140.0048 67.1576) (width 0.25) (layer "F.Cu") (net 17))
 (segment (start 158.9024 57.0992) (end 163.699 57.0992) (width 0.25) (layer "F.Cu") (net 17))
 (segment (start 174.0408 93.3704) (end 170.0276 97.3836) (width 0.25) (layer "F.Cu") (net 17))
 (segment (start 168.8592 103.3272) (end 141.5796 103.3272) (width 0.25) (layer "F.Cu") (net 17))
 (segment (start 158.9024 63.5992) (end 158.9024 57.0992) (width 0.25) (layer "F.Cu") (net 17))
 (segment (start 142.4432 64.7192) (end 151.5872 64.7192) (width 0.25) (layer "F.Cu") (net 17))
 (segment (start 160.02 64.7168) (end 158.9024 63.5992) (width 0.25) (layer "F.Cu") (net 17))
 (segment (start 175.6664 91.5416) (end 174.0408 91.5416) (width 0.25) (layer "F.Cu") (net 17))
 (segment (start 160.02 68.58) (end 160.02 64.7168) (width 0.25) (layer "F.Cu") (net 17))
 (segment (start 151.5872 64.7192) (end 155.448 68.58) (width 0.25) (layer "F.Cu") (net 17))
 (segment (start 163.699 57.0992) (end 164.0546 56.7436) (width 0.25) (layer "F.Cu") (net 17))
 (segment (start 174.0408 91.5416) (end 174.0408 93.3704) (width 0.25) (layer "F.Cu") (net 17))
 (segment (start 145.034 70.548) (end 142.4564 70.548) (width 0.25) (layer "F.Cu") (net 21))
 (segment (start 142.4564 70.548) (end 142.2908 70.7136) (width 0.25) (layer "F.Cu") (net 21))
 (segment (start 148.082 72.5424) (end 145.0396 72.5424) (width 0.25) (layer "F.Cu") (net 9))
 (segment (start 152.5631 71.6173) (end 152.5631 70.2564) (width 0.25) (layer "F.Cu") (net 9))
 (segment (start 151.638 72.5424) (end 152.5631 71.6173) (width 0.25) (layer "F.Cu") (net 9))
 (segment (start 148.082 72.5424) (end 151.638 72.5424) (width 0.25) (layer "F.Cu") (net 9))
 (segment (start 145.0396 72.5424) (end 145.034 72.548) (width 0.25) (layer "F.Cu") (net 9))
 (segment (start 152.6139 74.5236) (end 148.2344 74.5236) (width 0.25) (layer "F.Cu") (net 3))
 (segment (start 145.1112 74.6252) (end 145.034 74.548) (width 0.25) (layer "F.Cu") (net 3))
 (segment (start 148.1328 74.6252) (end 145.1112 74.6252) (width 0.25) (layer "F.Cu") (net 3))
 (segment (start 148.2344 74.5236) (end 148.1328 74.6252) (width 0.25) (layer "F.Cu") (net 3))
 (segment (start 171.6024 68.58) (end 171.9072 68.8848) (width 0.25) (layer "F.Cu") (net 12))
 (segment (start 171.9072 68.8848) (end 175.8884 68.8848) (width 0.25) (layer "F.Cu") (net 12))
 (segment (start 167.64 68.58) (end 171.6024 68.58) (width 0.25) (layer "F.Cu") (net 12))
 (segment (start 175.8884 68.8848) (end 176.1744 68.5988) (width 0.25) (layer "F.Cu") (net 12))
 (segment (start 175.6184 70.1548) (end 176.1744 69.5988) (width 0.25) (layer "F.Cu") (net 13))
 (segment (start 170.942 71.12) (end 171.9072 70.1548) (width 0.25) (layer "F.Cu") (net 13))
 (segment (start 167.64 71.12) (end 170.942 71.12) (width 0.25) (layer "F.Cu") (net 13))
 (segment (start 171.9072 70.1548) (end 175.6184 70.1548) (width 0.25) (layer "F.Cu") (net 13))
 (segment (start 166.1668 62.5856) (end 162.2044 66.548) (width 0.25) (layer "F.Cu") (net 15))
 (segment (start 177.8 64.4144) (end 175.9712 62.5856) (width 0.25) (layer "F.Cu") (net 15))
 (segment (start 175.9712 62.5856) (end 166.1668 62.5856) (width 0.25) (layer "F.Cu") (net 15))
 (segment (start 162.2044 77.9272) (end 161.3916 78.74) (width 0.25) (layer "F.Cu") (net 15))
 (segment (start 176.1744 72.6948) (end 177.8 71.0692) (width 0.25) (layer "F.Cu") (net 15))
 (segment (start 171.9072 72.6948) (end 176.1744 72.6948) (width 0.25) (layer "F.Cu") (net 15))
 (segment (start 161.3916 78.74) (end 160.02 78.74) (width 0.25) (layer "F.Cu") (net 15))
 (segment (start 177.8 71.0692) (end 177.8 64.4144) (width 0.25) (layer "F.Cu") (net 15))
 (segment (start 162.2044 66.548) (end 162.2044 77.9272) (width 0.25) (layer "F.Cu") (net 15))
 (segment (start 160.02 71.12) (end 156.3517 71.12) (width 0.25) (layer "F.Cu") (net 22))
 (segment (start 156.3517 71.12) (end 155.4881 70.2564) (width 0.25) (layer "F.Cu") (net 22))
 (segment (start 160.02 73.66) (end 156.4025 73.66) (width 0.25) (layer "F.Cu") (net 23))
 (segment (start 156.4025 73.66) (end 155.5389 74.5236) (width 0.25) (layer "F.Cu") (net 23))
 (segment (start 141.5288 90.5256) (end 142.8708 89.1836) (width 0.25) (layer "F.Cu") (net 4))
 (segment (start 141.5288 91.8571) (end 141.5288 90.5256) (width 0.25) (layer "F.Cu") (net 4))
 (segment (start 142.8708 89.1836) (end 142.8708 87.4752) (width 0.25) (layer "F.Cu") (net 4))
 (segment (start 158.9998 82.3002) (end 144.1958 82.3002) (width 0.25) (layer "F.Cu") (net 6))
 (segment (start 144.1958 82.3002) (end 142.8708 80.9752) (width 0.25) (layer "F.Cu") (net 6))
 (segment (start 160.02 81.28) (end 158.9998 82.3002) (width 0.25) (layer "F.Cu") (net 6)))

